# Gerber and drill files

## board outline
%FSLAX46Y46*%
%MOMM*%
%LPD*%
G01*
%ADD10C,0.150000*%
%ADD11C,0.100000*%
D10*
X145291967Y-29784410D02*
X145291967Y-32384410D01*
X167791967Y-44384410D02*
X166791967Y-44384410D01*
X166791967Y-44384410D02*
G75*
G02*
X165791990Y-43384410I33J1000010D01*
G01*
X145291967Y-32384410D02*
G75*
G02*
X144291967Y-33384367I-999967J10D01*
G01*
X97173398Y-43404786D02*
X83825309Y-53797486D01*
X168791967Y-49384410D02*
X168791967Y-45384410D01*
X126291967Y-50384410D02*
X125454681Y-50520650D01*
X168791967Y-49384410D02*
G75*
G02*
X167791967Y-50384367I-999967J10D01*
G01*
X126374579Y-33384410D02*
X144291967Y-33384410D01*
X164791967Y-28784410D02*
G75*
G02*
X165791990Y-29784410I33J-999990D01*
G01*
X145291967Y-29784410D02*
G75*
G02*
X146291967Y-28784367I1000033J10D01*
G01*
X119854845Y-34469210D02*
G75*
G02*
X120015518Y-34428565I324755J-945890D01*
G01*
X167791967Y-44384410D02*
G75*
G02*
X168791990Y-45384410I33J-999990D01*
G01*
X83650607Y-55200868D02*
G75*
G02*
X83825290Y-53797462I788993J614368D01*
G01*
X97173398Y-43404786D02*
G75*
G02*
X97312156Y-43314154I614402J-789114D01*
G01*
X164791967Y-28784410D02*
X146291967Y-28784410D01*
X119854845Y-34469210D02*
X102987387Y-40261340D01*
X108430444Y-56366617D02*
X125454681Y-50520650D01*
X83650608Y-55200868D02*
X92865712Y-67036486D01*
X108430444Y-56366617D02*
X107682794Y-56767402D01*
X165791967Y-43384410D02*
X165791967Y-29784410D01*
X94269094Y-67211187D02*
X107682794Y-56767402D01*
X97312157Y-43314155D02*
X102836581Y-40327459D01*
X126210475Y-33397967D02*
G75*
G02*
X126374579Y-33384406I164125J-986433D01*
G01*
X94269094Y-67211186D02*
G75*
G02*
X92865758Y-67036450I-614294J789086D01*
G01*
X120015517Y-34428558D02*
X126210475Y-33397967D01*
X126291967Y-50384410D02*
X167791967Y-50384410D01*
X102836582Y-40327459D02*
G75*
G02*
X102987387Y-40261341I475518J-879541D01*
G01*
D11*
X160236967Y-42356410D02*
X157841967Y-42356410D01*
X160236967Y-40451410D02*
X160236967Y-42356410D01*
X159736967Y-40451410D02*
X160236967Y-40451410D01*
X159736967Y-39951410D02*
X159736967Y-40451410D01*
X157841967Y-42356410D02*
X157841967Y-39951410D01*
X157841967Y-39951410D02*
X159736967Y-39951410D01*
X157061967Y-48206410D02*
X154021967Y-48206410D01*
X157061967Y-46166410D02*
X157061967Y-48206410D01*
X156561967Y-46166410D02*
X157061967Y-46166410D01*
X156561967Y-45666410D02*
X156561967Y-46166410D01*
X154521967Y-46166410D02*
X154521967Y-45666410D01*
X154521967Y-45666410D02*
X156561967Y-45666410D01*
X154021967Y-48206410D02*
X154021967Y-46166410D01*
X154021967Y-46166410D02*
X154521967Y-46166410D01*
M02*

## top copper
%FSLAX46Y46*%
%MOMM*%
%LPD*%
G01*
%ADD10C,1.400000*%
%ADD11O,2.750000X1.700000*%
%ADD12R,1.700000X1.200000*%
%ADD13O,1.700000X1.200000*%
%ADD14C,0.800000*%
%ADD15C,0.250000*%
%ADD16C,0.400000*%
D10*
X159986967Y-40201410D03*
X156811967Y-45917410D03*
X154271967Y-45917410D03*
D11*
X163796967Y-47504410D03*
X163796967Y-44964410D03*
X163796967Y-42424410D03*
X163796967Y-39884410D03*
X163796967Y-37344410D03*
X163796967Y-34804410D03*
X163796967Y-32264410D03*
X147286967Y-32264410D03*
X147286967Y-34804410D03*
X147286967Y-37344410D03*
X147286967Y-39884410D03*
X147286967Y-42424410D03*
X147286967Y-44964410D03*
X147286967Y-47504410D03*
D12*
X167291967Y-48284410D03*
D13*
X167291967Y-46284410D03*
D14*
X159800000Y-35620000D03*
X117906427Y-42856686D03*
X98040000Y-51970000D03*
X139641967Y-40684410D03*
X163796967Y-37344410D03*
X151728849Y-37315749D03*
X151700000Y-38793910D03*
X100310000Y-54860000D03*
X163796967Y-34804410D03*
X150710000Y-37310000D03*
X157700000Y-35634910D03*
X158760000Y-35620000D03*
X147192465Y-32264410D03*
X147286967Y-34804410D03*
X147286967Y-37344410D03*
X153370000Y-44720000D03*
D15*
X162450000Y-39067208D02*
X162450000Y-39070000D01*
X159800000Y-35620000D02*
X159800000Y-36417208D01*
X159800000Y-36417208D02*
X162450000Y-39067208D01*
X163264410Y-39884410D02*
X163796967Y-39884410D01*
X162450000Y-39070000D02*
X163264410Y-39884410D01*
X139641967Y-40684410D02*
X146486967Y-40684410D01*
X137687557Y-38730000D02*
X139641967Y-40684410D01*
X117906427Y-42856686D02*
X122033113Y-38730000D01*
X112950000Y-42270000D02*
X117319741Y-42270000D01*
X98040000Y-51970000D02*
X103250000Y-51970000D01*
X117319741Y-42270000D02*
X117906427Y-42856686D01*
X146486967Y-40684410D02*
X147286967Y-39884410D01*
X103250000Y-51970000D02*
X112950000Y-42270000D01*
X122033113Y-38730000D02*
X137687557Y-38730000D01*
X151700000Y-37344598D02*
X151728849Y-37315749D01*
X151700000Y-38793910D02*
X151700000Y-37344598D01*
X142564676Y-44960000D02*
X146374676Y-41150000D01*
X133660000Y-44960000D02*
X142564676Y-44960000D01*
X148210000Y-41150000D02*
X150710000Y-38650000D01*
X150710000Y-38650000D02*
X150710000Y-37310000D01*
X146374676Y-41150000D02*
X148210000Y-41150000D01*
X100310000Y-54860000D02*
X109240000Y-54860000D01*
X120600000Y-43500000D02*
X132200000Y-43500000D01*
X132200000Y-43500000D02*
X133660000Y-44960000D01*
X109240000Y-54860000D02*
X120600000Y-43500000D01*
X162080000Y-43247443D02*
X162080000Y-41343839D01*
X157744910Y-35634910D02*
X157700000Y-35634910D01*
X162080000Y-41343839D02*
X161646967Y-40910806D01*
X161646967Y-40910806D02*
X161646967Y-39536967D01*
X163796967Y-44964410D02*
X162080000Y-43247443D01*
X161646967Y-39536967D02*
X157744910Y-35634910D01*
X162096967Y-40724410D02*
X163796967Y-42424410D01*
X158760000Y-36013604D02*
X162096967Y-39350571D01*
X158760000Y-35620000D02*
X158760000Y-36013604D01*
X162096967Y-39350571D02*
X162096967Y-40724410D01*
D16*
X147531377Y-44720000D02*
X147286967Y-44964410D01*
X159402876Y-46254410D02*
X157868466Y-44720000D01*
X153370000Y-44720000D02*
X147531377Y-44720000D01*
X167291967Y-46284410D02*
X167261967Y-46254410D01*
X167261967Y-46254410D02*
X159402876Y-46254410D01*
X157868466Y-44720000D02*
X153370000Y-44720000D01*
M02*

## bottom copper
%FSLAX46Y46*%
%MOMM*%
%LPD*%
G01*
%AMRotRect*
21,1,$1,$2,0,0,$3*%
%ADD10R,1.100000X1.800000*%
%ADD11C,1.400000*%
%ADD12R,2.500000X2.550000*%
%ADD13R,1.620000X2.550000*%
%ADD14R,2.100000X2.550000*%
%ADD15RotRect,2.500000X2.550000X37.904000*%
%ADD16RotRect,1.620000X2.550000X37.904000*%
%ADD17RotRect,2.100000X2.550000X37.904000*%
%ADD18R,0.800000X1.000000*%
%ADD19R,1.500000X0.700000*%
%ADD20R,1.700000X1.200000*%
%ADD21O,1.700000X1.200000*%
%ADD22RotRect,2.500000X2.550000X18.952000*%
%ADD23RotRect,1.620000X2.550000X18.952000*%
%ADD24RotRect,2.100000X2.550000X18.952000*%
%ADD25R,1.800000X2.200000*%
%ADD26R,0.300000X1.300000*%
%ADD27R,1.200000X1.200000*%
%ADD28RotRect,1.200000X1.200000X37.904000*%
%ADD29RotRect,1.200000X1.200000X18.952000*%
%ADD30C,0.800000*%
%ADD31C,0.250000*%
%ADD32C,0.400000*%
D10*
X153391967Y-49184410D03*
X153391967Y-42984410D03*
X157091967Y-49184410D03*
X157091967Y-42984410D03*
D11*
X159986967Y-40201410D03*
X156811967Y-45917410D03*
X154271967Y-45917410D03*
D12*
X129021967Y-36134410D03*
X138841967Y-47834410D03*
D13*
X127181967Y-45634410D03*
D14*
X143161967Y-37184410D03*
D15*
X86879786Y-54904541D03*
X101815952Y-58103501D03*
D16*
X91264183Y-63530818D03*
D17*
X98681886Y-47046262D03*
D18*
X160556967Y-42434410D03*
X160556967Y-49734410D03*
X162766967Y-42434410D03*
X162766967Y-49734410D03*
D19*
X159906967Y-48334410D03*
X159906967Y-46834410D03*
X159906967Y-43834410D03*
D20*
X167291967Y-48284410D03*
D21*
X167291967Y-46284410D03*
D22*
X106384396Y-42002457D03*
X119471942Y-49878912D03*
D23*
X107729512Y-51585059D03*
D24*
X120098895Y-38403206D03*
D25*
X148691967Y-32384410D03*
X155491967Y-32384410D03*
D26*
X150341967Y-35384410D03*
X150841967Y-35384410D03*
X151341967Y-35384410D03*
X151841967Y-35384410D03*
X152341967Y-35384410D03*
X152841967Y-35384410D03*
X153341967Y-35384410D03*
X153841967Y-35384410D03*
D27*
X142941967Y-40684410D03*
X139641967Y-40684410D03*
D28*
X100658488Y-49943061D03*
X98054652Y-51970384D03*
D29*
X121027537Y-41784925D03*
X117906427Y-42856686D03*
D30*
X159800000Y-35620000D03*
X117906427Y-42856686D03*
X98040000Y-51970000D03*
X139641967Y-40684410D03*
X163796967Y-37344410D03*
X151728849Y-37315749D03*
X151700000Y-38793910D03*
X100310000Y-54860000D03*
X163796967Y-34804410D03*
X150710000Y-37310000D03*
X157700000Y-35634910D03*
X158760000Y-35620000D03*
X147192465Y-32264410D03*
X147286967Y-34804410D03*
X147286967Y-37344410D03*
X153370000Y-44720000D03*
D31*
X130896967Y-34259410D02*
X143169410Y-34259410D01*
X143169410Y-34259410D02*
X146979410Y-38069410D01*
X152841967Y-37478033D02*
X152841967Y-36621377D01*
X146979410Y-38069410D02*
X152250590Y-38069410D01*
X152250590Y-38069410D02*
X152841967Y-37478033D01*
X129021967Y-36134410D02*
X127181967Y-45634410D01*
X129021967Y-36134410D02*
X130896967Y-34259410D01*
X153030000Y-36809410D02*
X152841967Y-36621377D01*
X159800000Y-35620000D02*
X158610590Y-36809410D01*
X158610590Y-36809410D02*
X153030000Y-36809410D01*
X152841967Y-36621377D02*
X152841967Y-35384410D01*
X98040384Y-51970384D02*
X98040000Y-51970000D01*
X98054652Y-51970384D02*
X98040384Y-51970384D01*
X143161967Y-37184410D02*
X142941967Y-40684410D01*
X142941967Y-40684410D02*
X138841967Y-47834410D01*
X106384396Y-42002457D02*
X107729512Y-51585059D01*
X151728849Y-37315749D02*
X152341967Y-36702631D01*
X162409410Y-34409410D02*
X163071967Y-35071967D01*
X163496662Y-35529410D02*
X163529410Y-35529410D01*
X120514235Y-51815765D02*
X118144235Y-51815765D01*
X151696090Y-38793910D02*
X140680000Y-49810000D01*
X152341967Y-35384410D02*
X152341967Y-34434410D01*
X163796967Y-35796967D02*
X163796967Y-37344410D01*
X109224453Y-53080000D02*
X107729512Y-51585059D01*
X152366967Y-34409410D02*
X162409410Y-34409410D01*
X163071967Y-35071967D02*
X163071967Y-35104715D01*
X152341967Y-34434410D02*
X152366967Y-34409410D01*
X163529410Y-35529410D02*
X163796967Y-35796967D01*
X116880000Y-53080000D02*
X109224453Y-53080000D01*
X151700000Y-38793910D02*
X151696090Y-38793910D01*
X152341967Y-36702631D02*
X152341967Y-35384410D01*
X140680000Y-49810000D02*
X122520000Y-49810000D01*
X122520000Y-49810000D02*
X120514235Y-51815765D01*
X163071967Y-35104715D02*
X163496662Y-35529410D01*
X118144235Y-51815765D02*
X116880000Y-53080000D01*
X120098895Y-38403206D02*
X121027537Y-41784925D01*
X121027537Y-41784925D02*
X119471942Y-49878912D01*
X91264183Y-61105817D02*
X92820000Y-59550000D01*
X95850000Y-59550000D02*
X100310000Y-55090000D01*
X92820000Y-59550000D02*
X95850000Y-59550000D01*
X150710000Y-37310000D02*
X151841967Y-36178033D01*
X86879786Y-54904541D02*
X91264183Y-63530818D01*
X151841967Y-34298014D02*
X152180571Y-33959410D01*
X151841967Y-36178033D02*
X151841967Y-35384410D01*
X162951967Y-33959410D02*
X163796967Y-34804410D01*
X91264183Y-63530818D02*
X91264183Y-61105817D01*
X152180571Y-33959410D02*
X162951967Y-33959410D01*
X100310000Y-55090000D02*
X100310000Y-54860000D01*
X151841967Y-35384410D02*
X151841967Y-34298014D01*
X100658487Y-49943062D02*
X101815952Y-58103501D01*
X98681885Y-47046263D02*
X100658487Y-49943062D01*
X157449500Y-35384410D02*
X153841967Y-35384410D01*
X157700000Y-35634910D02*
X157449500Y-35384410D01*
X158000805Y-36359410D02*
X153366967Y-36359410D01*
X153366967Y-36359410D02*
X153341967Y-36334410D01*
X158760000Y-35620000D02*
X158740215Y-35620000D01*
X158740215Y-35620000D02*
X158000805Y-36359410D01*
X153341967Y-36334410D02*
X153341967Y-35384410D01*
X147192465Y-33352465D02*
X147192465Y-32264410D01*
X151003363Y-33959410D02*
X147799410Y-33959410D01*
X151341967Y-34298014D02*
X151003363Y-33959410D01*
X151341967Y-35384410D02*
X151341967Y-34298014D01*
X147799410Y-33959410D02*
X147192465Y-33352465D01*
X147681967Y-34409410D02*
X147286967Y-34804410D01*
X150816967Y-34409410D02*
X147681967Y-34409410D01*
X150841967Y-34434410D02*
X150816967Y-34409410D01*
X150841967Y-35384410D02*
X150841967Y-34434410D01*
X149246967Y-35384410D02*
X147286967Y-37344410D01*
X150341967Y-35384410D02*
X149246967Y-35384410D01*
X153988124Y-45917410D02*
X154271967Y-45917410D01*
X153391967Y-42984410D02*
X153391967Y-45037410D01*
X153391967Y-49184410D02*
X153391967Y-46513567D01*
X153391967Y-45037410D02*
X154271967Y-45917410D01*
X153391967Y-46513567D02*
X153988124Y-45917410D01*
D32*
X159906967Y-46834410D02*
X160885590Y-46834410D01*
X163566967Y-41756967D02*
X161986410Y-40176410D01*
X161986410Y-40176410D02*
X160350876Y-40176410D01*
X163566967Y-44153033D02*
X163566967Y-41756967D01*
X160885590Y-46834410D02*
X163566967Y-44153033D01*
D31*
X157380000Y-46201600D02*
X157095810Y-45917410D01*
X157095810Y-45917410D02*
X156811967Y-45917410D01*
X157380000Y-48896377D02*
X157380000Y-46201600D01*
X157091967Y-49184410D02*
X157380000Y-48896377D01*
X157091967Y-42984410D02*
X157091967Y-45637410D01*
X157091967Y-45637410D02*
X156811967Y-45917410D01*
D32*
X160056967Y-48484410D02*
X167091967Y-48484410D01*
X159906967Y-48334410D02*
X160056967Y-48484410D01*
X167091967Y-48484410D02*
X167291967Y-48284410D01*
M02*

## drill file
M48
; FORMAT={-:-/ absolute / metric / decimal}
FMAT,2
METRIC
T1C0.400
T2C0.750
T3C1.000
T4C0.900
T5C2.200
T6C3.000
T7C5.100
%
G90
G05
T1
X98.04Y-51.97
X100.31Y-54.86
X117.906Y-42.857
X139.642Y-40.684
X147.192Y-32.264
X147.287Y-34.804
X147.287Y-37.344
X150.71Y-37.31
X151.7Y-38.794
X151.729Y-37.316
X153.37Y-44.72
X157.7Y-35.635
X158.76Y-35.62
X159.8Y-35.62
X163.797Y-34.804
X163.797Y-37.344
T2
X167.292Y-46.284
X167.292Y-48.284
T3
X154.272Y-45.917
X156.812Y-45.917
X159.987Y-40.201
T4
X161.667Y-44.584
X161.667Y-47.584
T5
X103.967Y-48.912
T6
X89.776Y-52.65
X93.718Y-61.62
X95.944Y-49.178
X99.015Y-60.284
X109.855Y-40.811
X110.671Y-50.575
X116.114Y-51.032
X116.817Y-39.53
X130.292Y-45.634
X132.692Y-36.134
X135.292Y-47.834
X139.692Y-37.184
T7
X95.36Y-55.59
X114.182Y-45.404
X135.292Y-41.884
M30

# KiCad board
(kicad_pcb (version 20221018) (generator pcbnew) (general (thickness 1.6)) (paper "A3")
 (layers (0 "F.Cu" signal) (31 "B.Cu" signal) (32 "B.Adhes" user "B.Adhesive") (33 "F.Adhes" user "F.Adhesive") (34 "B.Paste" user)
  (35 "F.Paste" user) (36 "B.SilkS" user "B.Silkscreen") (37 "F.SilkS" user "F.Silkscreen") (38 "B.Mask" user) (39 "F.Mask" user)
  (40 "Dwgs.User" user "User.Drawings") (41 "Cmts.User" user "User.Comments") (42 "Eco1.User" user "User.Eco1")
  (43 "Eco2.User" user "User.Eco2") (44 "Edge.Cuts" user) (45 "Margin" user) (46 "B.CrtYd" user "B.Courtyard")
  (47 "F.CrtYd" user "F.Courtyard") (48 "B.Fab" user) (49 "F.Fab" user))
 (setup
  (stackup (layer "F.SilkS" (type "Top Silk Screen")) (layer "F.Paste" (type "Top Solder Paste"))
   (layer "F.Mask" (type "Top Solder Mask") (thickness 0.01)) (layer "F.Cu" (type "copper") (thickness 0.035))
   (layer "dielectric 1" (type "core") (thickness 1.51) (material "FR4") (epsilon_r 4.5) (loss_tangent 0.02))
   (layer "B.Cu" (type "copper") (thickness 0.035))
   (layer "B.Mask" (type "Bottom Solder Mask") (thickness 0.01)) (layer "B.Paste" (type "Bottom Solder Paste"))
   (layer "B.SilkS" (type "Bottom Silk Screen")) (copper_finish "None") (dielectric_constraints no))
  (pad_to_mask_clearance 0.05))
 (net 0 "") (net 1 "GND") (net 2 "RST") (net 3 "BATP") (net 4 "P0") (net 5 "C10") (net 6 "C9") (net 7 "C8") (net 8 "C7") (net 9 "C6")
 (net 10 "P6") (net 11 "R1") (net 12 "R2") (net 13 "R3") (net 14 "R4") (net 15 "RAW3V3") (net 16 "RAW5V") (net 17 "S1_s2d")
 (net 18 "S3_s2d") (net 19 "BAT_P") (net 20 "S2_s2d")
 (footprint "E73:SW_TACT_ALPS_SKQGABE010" (layer "F.Cu") (at 155.241967 46.08441 90)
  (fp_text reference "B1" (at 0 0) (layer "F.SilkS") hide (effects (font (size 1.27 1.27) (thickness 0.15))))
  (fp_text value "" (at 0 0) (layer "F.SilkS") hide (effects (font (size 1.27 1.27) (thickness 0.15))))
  (pad "1" smd rect (at -3.1 -1.85 90) (size 1.8 1.1) (layers "B.Cu" "B.Paste" "B.Mask") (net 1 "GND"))
  (pad "1" smd rect (at 3.1 -1.85 90) (size 1.8 1.1) (layers "B.Cu" "B.Paste" "B.Mask") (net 1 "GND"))
  (pad "2" smd rect (at -3.1 1.85 90) (size 1.8 1.1) (layers "B.Cu" "B.Paste" "B.Mask") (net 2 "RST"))
  (pad "2" smd rect (at 3.1 1.85 90) (size 1.8 1.1) (layers "B.Cu" "B.Paste" "B.Mask") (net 2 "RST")))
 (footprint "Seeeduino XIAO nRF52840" (layer "F.Cu") (at 155.541967 39.88441 180)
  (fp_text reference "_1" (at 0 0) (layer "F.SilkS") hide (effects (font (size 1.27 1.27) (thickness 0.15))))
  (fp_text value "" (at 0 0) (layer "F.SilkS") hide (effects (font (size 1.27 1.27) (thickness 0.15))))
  (fp_line (start -4.695 -2.472) (end -2.3 -2.472) (stroke (width 0.1) (type solid)) (layer "Edge.Cuts"))
  (fp_line (start -4.695 -0.567) (end -4.695 -2.472) (stroke (width 0.1) (type solid)) (layer "Edge.Cuts"))
  (fp_line (start -4.195 -0.567) (end -4.695 -0.567) (stroke (width 0.1) (type solid)) (layer "Edge.Cuts"))
  (fp_line (start -4.195 -0.067) (end -4.195 -0.567) (stroke (width 0.1) (type solid)) (layer "Edge.Cuts"))
  (fp_line (start -2.3 -2.472) (end -2.3 -0.067) (stroke (width 0.1) (type solid)) (layer "Edge.Cuts"))
  (fp_line (start -2.3 -0.067) (end -4.195 -0.067) (stroke (width 0.1) (type solid)) (layer "Edge.Cuts"))
  (fp_line (start -1.52 -8.322) (end 1.52 -8.322) (stroke (width 0.1) (type solid)) (layer "Edge.Cuts"))
  (fp_line (start -1.52 -6.282) (end -1.52 -8.322) (stroke (width 0.1) (type solid)) (layer "Edge.Cuts"))
  (fp_line (start -1.02 -6.282) (end -1.52 -6.282) (stroke (width 0.1) (type solid)) (layer "Edge.Cuts"))
  (fp_line (start -1.02 -5.782) (end -1.02 -6.282) (stroke (width 0.1) (type solid)) (layer "Edge.Cuts"))
  (fp_line (start 1.02 -6.282) (end 1.02 -5.782) (stroke (width 0.1) (type solid)) (layer "Edge.Cuts"))
  (fp_line (start 1.02 -5.782) (end -1.02 -5.782) (stroke (width 0.1) (type solid)) (layer "Edge.Cuts"))
  (fp_line (start 1.52 -8.322) (end 1.52 -6.282) (stroke (width 0.1) (type solid)) (layer "Edge.Cuts"))
  (fp_line (start 1.52 -6.282) (end 1.02 -6.282) (stroke (width 0.1) (type solid)) (layer "Edge.Cuts"))
  (pad "" thru_hole circle (at -4.445 -0.317) (size 1.4 1.4) (drill 1) (layers "*.Cu" "*.Mask") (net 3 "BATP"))
  (pad "" thru_hole circle (at -1.27 -6.033) (size 1.4 1.4) (drill 1) (layers "*.Cu" "*.Mask") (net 2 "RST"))
  (pad "" thru_hole circle (at 1.27 -6.033) (size 1.4 1.4) (drill 1) (layers "*.Cu" "*.Mask") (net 1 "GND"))
  (pad "1" smd oval (at -8.255 -7.62 180) (size 2.75 1.7) (layers "F.Cu" "F.Paste" "F.Mask") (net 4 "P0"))
  (pad "2" smd oval (at -8.255 -5.08 180) (size 2.75 1.7) (layers "F.Cu" "F.Paste" "F.Mask") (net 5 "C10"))
  (pad "3" smd oval (at -8.255 -2.54 180) (size 2.75 1.7) (layers "F.Cu" "F.Paste" "F.Mask") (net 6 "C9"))
  (pad "4" smd oval (at -8.255 0 180) (size 2.75 1.7) (layers "F.Cu" "F.Paste" "F.Mask") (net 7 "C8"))
  (pad "5" smd oval (at -8.255 2.54 180) (size 2.75 1.7) (layers "F.Cu" "F.Paste" "F.Mask") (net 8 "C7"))
  (pad "6" smd oval (at -8.255 5.08 180) (size 2.75 1.7) (layers "F.Cu" "F.Paste" "F.Mask") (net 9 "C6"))
  (pad "7" smd oval (at -8.255 7.62 180) (size 2.75 1.7) (layers "F.Cu" "F.Paste" "F.Mask") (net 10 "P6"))
  (pad "8" smd oval (at 8.255 7.62 180) (size 2.75 1.7) (layers "F.Cu" "F.Paste" "F.Mask") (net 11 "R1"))
  (pad "9" smd oval (at 8.255 5.08 180) (size 2.75 1.7) (layers "F.Cu" "F.Paste" "F.Mask") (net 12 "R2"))
  (pad "10" smd oval (at 8.255 2.54 180) (size 2.75 1.7) (layers "F.Cu" "F.Paste" "F.Mask") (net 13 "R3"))
  (pad "11" smd oval (at 8.255 0 180) (size 2.75 1.7) (layers "F.Cu" "F.Paste" "F.Mask") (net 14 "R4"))
  (pad "12" smd oval (at 8.255 -2.54 180) (size 2.75 1.7) (layers "F.Cu" "F.Paste" "F.Mask") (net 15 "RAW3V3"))
  (pad "13" smd oval (at 8.255 -5.08 180) (size 2.75 1.7) (layers "F.Cu" "F.Paste" "F.Mask") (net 1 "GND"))
  (pad "14" smd oval (at 8.255 -7.62 180) (size 2.75 1.7) (layers "F.Cu" "F.Paste" "F.Mask") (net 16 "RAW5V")))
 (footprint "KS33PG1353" (layer "F.Cu") (at 135.291967 41.88441)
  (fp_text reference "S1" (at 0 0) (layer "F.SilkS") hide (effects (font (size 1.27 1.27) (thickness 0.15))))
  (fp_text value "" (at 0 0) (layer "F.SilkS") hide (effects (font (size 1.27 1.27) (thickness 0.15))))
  (pad "" np_thru_hole circle (at -5 3.75) (size 3 3) (drill 3) (layers "*.Cu" "*.Mask"))
  (pad "" np_thru_hole circle (at -2.6 -5.75) (size 3 3) (drill 3) (layers "*.Cu" "*.Mask"))
  (pad "" np_thru_hole circle (at 0 0) (size 5.1 5.1) (drill 5.1) (layers "*.Cu" "*.Mask"))
  (pad "" np_thru_hole circle (at 0 5.95) (size 3 3) (drill 3) (layers "*.Cu" "*.Mask"))
  (pad "" np_thru_hole circle (at 4.4 -4.7) (size 3 3) (drill 3) (layers "*.Cu" "*.Mask"))
  (pad "1" smd rect (at -6.27 -5.75) (size 2.5 2.55) (layers "B.Cu" "B.Paste" "B.Mask") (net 7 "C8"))
  (pad "1" smd rect (at 3.55 5.95) (size 2.5 2.55) (layers "B.Cu" "B.Paste" "B.Mask") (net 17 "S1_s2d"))
  (pad "2" smd rect (at -8.11 3.75) (size 1.62 2.55) (layers "B.Cu" "B.Paste" "B.Mask") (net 7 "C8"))
  (pad "2" smd rect (at 7.87 -4.7) (size 2.1 2.55) (layers "B.Cu" "B.Paste" "B.Mask") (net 17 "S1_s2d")))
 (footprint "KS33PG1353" (layer "F.Cu") (at 95.359531 55.589614 37.904)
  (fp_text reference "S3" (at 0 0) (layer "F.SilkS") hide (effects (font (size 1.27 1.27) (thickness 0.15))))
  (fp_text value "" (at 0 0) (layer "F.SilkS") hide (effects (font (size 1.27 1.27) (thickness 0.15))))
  (pad "" np_thru_hole circle (at -5 3.75) (size 3 3) (drill 3) (layers "*.Cu" "*.Mask"))
  (pad "" np_thru_hole circle (at -2.6 -5.75) (size 3 3) (drill 3) (layers "*.Cu" "*.Mask"))
  (pad "" np_thru_hole circle (at 0 0) (size 5.1 5.1) (drill 5.1) (layers "*.Cu" "*.Mask"))
  (pad "" np_thru_hole circle (at 0 5.95) (size 3 3) (drill 3) (layers "*.Cu" "*.Mask"))
  (pad "" np_thru_hole circle (at 4.4 -4.7) (size 3 3) (drill 3) (layers "*.Cu" "*.Mask"))
  (pad "1" smd rect (at -6.27 -5.75 37.904) (size 2.5 2.55) (layers "B.Cu" "B.Paste" "B.Mask") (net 9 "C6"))
  (pad "1" smd rect (at 3.55 5.95 37.904) (size 2.5 2.55) (layers "B.Cu" "B.Paste" "B.Mask") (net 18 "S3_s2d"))
  (pad "2" smd rect (at -8.11 3.75 37.904) (size 1.62 2.55) (layers "B.Cu" "B.Paste" "B.Mask") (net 9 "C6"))
  (pad "2" smd rect (at 7.87 -4.7 37.904) (size 2.1 2.55) (layers "B.Cu" "B.Paste" "B.Mask") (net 18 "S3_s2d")))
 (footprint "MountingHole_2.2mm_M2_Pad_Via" (layer "F.Cu") (at 103.967424 48.91199 18.952)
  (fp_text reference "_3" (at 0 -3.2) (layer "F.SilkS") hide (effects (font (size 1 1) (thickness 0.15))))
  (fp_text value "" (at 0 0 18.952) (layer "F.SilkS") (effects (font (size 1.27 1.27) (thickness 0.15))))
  (pad "" np_thru_hole circle (at 0 0) (size 2.2 2.2) (drill 2.2) (layers "*.Cu" "*.Mask")))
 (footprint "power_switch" (layer "F.Cu") (at 161.641967 46.08441)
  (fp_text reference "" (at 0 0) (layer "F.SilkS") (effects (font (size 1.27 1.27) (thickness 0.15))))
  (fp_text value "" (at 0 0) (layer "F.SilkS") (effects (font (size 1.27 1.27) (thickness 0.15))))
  (pad "" smd rect (at -1.085 -3.65 270) (size 1 0.8) (layers "B.Cu" "B.Paste" "B.Mask"))
  (pad "" smd rect (at -1.085 3.65 270) (size 1 0.8) (layers "B.Cu" "B.Paste" "B.Mask"))
  (pad "" np_thru_hole circle (at 0.025 -1.5 90) (size 0.9 0.9) (drill 0.9) (layers "*.Cu" "*.Mask"))
  (pad "" np_thru_hole circle (at 0.025 1.5 90) (size 0.9 0.9) (drill 0.9) (layers "*.Cu" "*.Mask"))
  (pad "" smd rect (at 1.125 -3.65 270) (size 1 0.8) (layers "B.Cu" "B.Paste" "B.Mask"))
  (pad "" smd rect (at 1.125 3.65 270) (size 1 0.8) (layers "B.Cu" "B.Paste" "B.Mask"))
  (pad "4" smd rect (at -1.735 2.25 270) (size 0.7 1.5) (layers "B.Cu" "B.Paste" "B.Mask") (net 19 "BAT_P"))
  (pad "5" smd rect (at -1.735 0.75 270) (size 0.7 1.5) (layers "B.Cu" "B.Paste" "B.Mask") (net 3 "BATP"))
  (pad "6" smd rect (at -1.735 -2.25 270) (size 0.7 1.5) (layers "B.Cu" "B.Paste" "B.Mask")))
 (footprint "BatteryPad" (layer "F.Cu") (at 167.291967 47.28441 90)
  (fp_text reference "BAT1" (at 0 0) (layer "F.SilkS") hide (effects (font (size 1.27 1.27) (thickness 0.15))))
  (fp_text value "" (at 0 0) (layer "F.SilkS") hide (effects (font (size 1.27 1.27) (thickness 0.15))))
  (pad "1" thru_hole rect (at -1 0 90) (size 1.2 1.7) (drill 0.75) (layers "*.Cu" "*.Mask") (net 19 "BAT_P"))
  (pad "2" thru_hole oval (at 1 0 90) (size 1.2 1.7) (drill 0.75) (layers "*.Cu" "*.Mask") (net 1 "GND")))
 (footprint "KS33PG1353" (layer "F.Cu") (at 114.181967 45.40441 18.952)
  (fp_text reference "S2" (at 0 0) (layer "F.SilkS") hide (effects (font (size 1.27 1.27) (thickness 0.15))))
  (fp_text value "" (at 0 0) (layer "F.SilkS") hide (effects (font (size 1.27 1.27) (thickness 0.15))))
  (pad "" np_thru_hole circle (at -5 3.75) (size 3 3) (drill 3) (layers "*.Cu" "*.Mask"))
  (pad "" np_thru_hole circle (at -2.6 -5.75) (size 3 3) (drill 3) (layers "*.Cu" "*.Mask"))
  (pad "" np_thru_hole circle (at 0 0) (size 5.1 5.1) (drill 5.1) (layers "*.Cu" "*.Mask"))
  (pad "" np_thru_hole circle (at 0 5.95) (size 3 3) (drill 3) (layers "*.Cu" "*.Mask"))
  (pad "" np_thru_hole circle (at 4.4 -4.7) (size 3 3) (drill 3) (layers "*.Cu" "*.Mask"))
  (pad "1" smd rect (at -6.27 -5.75 18.952) (size 2.5 2.55) (layers "B.Cu" "B.Paste" "B.Mask") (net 8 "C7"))
  (pad "1" smd rect (at 3.55 5.95 18.952) (size 2.5 2.55) (layers "B.Cu" "B.Paste" "B.Mask") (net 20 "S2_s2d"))
  (pad "2" smd rect (at -8.11 3.75 18.952) (size 1.62 2.55) (layers "B.Cu" "B.Paste" "B.Mask") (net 8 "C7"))
  (pad "2" smd rect (at 7.87 -4.7 18.952) (size 2.1 2.55) (layers "B.Cu" "B.Paste" "B.Mask") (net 20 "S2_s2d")))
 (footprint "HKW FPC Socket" (layer "B.Cu") (at 152.091967 32.38441)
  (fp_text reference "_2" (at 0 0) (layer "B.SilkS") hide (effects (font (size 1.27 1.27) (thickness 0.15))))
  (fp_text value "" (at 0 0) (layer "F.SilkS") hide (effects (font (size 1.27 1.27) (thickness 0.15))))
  (pad "" smd rect (at -3.4 0) (size 1.8 2.2) (layers "B.Cu" "B.Paste" "B.Mask"))
  (pad "" smd rect (at 3.4 0) (size 1.8 2.2) (layers "B.Cu" "B.Paste" "B.Mask"))
  (pad "1" smd rect (at -1.75 3) (size 0.3 1.3) (layers "B.Cu" "B.Paste" "B.Mask") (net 13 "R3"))
  (pad "2" smd rect (at -1.25 3) (size 0.3 1.3) (layers "B.Cu" "B.Paste" "B.Mask") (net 12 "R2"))
  (pad "3" smd rect (at -0.75 3) (size 0.3 1.3) (layers "B.Cu" "B.Paste" "B.Mask") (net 11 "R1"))
  (pad "4" smd rect (at -0.25 3) (size 0.3 1.3) (layers "B.Cu" "B.Paste" "B.Mask") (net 9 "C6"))
  (pad "5" smd rect (at 0.25 3) (size 0.3 1.3) (layers "B.Cu" "B.Paste" "B.Mask") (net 8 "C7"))
  (pad "6" smd rect (at 0.75 3) (size 0.3 1.3) (layers "B.Cu" "B.Paste" "B.Mask") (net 7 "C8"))
  (pad "7" smd rect (at 1.25 3) (size 0.3 1.3) (layers "B.Cu" "B.Paste" "B.Mask") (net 6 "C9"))
  (pad "8" smd rect (at 1.75 3) (size 0.3 1.3) (layers "B.Cu" "B.Paste" "B.Mask") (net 5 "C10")))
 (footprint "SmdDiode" (layer "B.Cu") (at 135.291967 41.88441)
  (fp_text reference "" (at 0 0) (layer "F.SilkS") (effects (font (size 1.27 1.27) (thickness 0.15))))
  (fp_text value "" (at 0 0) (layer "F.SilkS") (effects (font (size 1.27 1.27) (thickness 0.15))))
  (pad "1" smd rect (at 7.65 -1.2) (size 1.2 1.2) (layers "B.Cu" "B.Paste" "B.Mask") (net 17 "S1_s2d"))
  (pad "2" smd rect (at 4.35 -1.2) (size 1.2 1.2) (layers "B.Cu" "B.Paste" "B.Mask") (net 14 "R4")))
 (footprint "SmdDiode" (layer "B.Cu") (at 95.359531 55.589614 37.904)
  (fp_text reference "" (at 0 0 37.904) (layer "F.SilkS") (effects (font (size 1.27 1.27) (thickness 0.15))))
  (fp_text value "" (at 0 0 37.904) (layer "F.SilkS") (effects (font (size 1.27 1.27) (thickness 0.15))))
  (pad "1" smd rect (at 7.65 -1.2 37.904) (size 1.2 1.2) (layers "B.Cu" "B.Paste" "B.Mask") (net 18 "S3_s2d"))
  (pad "2" smd rect (at 4.35 -1.2 37.904) (size 1.2 1.2) (layers "B.Cu" "B.Paste" "B.Mask") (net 14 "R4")))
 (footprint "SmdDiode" (layer "B.Cu") (at 114.181967 45.40441 18.952)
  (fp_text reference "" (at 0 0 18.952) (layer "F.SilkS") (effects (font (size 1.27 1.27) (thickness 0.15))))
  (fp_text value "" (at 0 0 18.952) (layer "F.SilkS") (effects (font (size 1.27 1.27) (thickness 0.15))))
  (pad "1" smd rect (at 7.65 -1.2 18.952) (size 1.2 1.2) (layers "B.Cu" "B.Paste" "B.Mask") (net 20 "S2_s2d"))
  (pad "2" smd rect (at 4.35 -1.2 18.952) (size 1.2 1.2) (layers "B.Cu" "B.Paste" "B.Mask") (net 14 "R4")))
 (gr_line (start 145.291967 29.78441) (end 145.291967 32.38441) (stroke (width 0.15) (type solid)) (layer "Edge.Cuts"))
 (gr_line (start 167.791967 44.38441) (end 166.791967 44.38441) (stroke (width 0.15) (type solid)) (layer "Edge.Cuts"))
 (gr_arc (start 166.791967 44.38441) (mid 166.08486 44.091517) (end 165.791967 43.38441) (stroke (width 0.15) (type solid))
  (layer "Edge.Cuts"))
 (gr_arc (start 145.291967 32.38441) (mid 144.999074 33.091517) (end 144.291967 33.38441) (stroke (width 0.15) (type solid))
  (layer "Edge.Cuts"))
 (gr_line (start 97.173398 43.404786) (end 83.825309 53.797486) (stroke (width 0.15) (type solid)) (layer "Edge.Cuts"))
 (gr_line (start 168.791967 49.38441) (end 168.791967 45.38441) (stroke (width 0.15) (type solid)) (layer "Edge.Cuts"))
 (gr_line (start 126.291967 50.38441) (end 125.454681 50.52065) (stroke (width 0.15) (type solid)) (layer "Edge.Cuts"))
 (gr_arc (start 168.791967 49.38441) (mid 168.499074 50.091517) (end 167.791967 50.38441) (stroke (width 0.15) (type solid))
  (layer "Edge.Cuts"))
 (gr_line (start 126.374579 33.38441) (end 144.291967 33.38441) (stroke (width 0.15) (type solid)) (layer "Edge.Cuts"))
 (gr_arc (start 164.791967 28.78441) (mid 165.499074 29.077303) (end 165.791967 29.78441) (stroke (width 0.15) (type solid))
  (layer "Edge.Cuts"))
 (gr_arc (start 145.291967 29.78441) (mid 145.58486 29.077303) (end 146.291967 28.78441) (stroke (width 0.15) (type solid))
  (layer "Edge.Cuts"))
 (gr_arc (start 119.854845 34.46921) (mid 119.934337 34.44555) (end 120.015517 34.428558) (stroke (width 0.15) (type solid))
  (layer "Edge.Cuts"))
 (gr_arc (start 167.791967 44.38441) (mid 168.499074 44.677303) (end 168.791967 45.38441) (stroke (width 0.15) (type solid))
  (layer "Edge.Cuts"))
 (gr_arc (start 83.650607 55.200868) (mid 83.447308 54.462995) (end 83.825309 53.797486) (stroke (width 0.15) (type solid))
  (layer "Edge.Cuts"))
 (gr_arc (start 97.173398 43.404786) (mid 97.240897 43.356591) (end 97.312157 43.314155) (stroke (width 0.15) (type solid))
  (layer "Edge.Cuts"))
 (gr_line (start 164.791967 28.78441) (end 146.291967 28.78441) (stroke (width 0.15) (type solid)) (layer "Edge.Cuts"))
 (gr_line (start 119.854845 34.46921) (end 102.987387 40.26134) (stroke (width 0.15) (type solid)) (layer "Edge.Cuts"))
 (gr_line (start 108.430444 56.366617) (end 125.454681 50.52065) (stroke (width 0.15) (type solid)) (layer "Edge.Cuts"))
 (gr_line (start 83.650608 55.200868) (end 92.865712 67.036486) (stroke (width 0.15) (type solid)) (layer "Edge.Cuts"))
 (gr_line (start 108.430444 56.366617) (end 107.682794 56.767402) (stroke (width 0.15) (type solid)) (layer "Edge.Cuts"))
 (gr_line (start 165.791967 43.38441) (end 165.791967 29.78441) (stroke (width 0.15) (type solid)) (layer "Edge.Cuts"))
 (gr_line (start 94.269094 67.211187) (end 107.682794 56.767402) (stroke (width 0.15) (type solid)) (layer "Edge.Cuts"))
 (gr_line (start 97.312157 43.314155) (end 102.836581 40.327459) (stroke (width 0.15) (type solid)) (layer "Edge.Cuts"))
 (gr_arc (start 126.210475 33.397967) (mid 126.292247 33.387805) (end 126.374579 33.38441) (stroke (width 0.15) (type solid))
  (layer "Edge.Cuts"))
 (gr_arc (start 94.269094 67.211186) (mid 93.531221 67.414486) (end 92.865712 67.036486) (stroke (width 0.15) (type solid))
  (layer "Edge.Cuts"))
 (gr_line (start 120.015517 34.428558) (end 126.210475 33.397967) (stroke (width 0.15) (type solid)) (layer "Edge.Cuts"))
 (gr_line (start 126.291967 50.38441) (end 167.791967 50.38441) (stroke (width 0.15) (type solid)) (layer "Edge.Cuts"))
 (gr_arc (start 102.836582 40.327459) (mid 102.910621 40.29129) (end 102.987387 40.26134) (stroke (width 0.15) (type solid))
  (layer "Edge.Cuts"))
 (segment (start 162.45 39.067208) (end 162.45 39.07) (width 0.25) (layer "F.Cu") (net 7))
 (segment (start 159.8 35.62) (end 159.8 36.417208) (width 0.25) (layer "F.Cu") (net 7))
 (segment (start 159.8 36.417208) (end 162.45 39.067208) (width 0.25) (layer "F.Cu") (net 7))
 (segment (start 163.26441 39.88441) (end 163.796967 39.88441) (width 0.25) (layer "F.Cu") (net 7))
 (segment (start 162.45 39.07) (end 163.26441 39.88441) (width 0.25) (layer "F.Cu") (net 7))
 (via (at 159.8 35.62) (size 0.8) (drill 0.4) (layers "F.Cu" "B.Cu") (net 7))
 (segment (start 130.896967 34.25941) (end 143.16941 34.25941) (width 0.25) (layer "B.Cu") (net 7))
 (segment (start 143.16941 34.25941) (end 146.97941 38.06941) (width 0.25) (layer "B.Cu") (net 7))
 (segment (start 152.841967 37.478033) (end 152.841967 36.621377) (width 0.25) (layer "B.Cu") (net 7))
 (segment (start 146.97941 38.06941) (end 152.25059 38.06941) (width 0.25) (layer "B.Cu") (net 7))
 (segment (start 152.25059 38.06941) (end 152.841967 37.478033) (width 0.25) (layer "B.Cu") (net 7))
 (segment (start 129.021967 36.13441) (end 127.181967 45.63441) (width 0.25) (layer "B.Cu") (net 7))
 (segment (start 129.021967 36.13441) (end 130.896967 34.25941) (width 0.25) (layer "B.Cu") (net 7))
 (segment (start 153.03 36.80941) (end 152.841967 36.621377) (width 0.25) (layer "B.Cu") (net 7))
 (segment (start 159.8 35.62) (end 158.61059 36.80941) (width 0.25) (layer "B.Cu") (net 7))
 (segment (start 158.61059 36.80941) (end 153.03 36.80941) (width 0.25) (layer "B.Cu") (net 7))
 (segment (start 152.841967 36.621377) (end 152.841967 35.38441) (width 0.25) (layer "B.Cu") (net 7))
 (segment (start 139.641967 40.68441) (end 146.486967 40.68441) (width 0.25) (layer "F.Cu") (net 14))
 (segment (start 137.687557 38.73) (end 139.641967 40.68441) (width 0.25) (layer "F.Cu") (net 14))
 (segment (start 117.906427 42.856686) (end 122.033113 38.73) (width 0.25) (layer "F.Cu") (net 14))
 (segment (start 112.95 42.27) (end 117.319741 42.27) (width 0.25) (layer "F.Cu") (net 14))
 (segment (start 98.04 51.97) (end 103.25 51.97) (width 0.25) (layer "F.Cu") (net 14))
 (segment (start 117.319741 42.27) (end 117.906427 42.856686) (width 0.25) (layer "F.Cu") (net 14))
 (segment (start 146.486967 40.68441) (end 147.286967 39.88441) (width 0.25) (layer "F.Cu") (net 14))
 (segment (start 103.25 51.97) (end 112.95 42.27) (width 0.25) (layer "F.Cu") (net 14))
 (segment (start 122.033113 38.73) (end 137.687557 38.73) (width 0.25) (layer "F.Cu") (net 14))
 (via (at 117.906427 42.856686) (size 0.8) (drill 0.4) (layers "F.Cu" "B.Cu") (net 14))
 (via (at 98.04 51.97) (size 0.8) (drill 0.4) (layers "F.Cu" "B.Cu") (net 14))
 (via (at 139.641967 40.68441) (size 0.8) (drill 0.4) (layers "F.Cu" "B.Cu") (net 14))
 (segment (start 98.040384 51.970384) (end 98.04 51.97) (width 0.25) (layer "B.Cu") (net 14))
 (segment (start 98.054652 51.970384) (end 98.040384 51.970384) (width 0.25) (layer "B.Cu") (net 14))
 (segment (start 143.161967 37.18441) (end 142.941967 40.68441) (width 0.25) (layer "B.Cu") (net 17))
 (segment (start 142.941967 40.68441) (end 138.841967 47.83441) (width 0.25) (layer "B.Cu") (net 17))
 (segment (start 151.7 37.344598) (end 151.728849 37.315749) (width 0.25) (layer "F.Cu") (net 8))
 (segment (start 151.7 38.79391) (end 151.7 37.344598) (width 0.25) (layer "F.Cu") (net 8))
 (via (at 163.796967 37.34441) (size 0.8) (drill 0.4) (layers "F.Cu" "B.Cu") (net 8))
 (via (at 151.728849 37.315749) (size 0.8) (drill 0.4) (layers "F.Cu" "B.Cu") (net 8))
 (via (at 151.7 38.79391) (size 0.8) (drill 0.4) (layers "F.Cu" "B.Cu") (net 8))
 (segment (start 106.384396 42.002457) (end 107.729512 51.585059) (width 0.25) (layer "B.Cu") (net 8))
 (segment (start 151.728849 37.315749) (end 152.341967 36.702631) (width 0.25) (layer "B.Cu") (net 8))
 (segment (start 162.40941 34.40941) (end 163.071967 35.071967) (width 0.25) (layer "B.Cu") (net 8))
 (segment (start 163.496662 35.52941) (end 163.52941 35.52941) (width 0.25) (layer "B.Cu") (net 8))
 (segment (start 120.514235 51.815765) (end 118.144235 51.815765) (width 0.25) (layer "B.Cu") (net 8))
 (segment (start 151.69609 38.79391) (end 140.68 49.81) (width 0.25) (layer "B.Cu") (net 8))
 (segment (start 152.341967 35.38441) (end 152.341967 34.43441) (width 0.25) (layer "B.Cu") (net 8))
 (segment (start 163.796967 35.796967) (end 163.796967 37.34441) (width 0.25) (layer "B.Cu") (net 8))
 (segment (start 109.224453 53.08) (end 107.729512 51.585059) (width 0.25) (layer "B.Cu") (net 8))
 (segment (start 152.366967 34.40941) (end 162.40941 34.40941) (width 0.25) (layer "B.Cu") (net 8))
 (segment (start 163.071967 35.071967) (end 163.071967 35.104715) (width 0.25) (layer "B.Cu") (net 8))
 (segment (start 152.341967 34.43441) (end 152.366967 34.40941) (width 0.25) (layer "B.Cu") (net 8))
 (segment (start 163.52941 35.52941) (end 163.796967 35.796967) (width 0.25) (layer "B.Cu") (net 8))
 (segment (start 116.88 53.08) (end 109.224453 53.08) (width 0.25) (layer "B.Cu") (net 8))
 (segment (start 151.7 38.79391) (end 151.69609 38.79391) (width 0.25) (layer "B.Cu") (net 8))
 (segment (start 152.341967 36.702631) (end 152.341967 35.38441) (width 0.25) (layer "B.Cu") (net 8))
 (segment (start 140.68 49.81) (end 122.52 49.81) (width 0.25) (layer "B.Cu") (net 8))
 (segment (start 122.52 49.81) (end 120.514235 51.815765) (width 0.25) (layer "B.Cu") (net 8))
 (segment (start 163.071967 35.104715) (end 163.496662 35.52941) (width 0.25) (layer "B.Cu") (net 8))
 (segment (start 118.144235 51.815765) (end 116.88 53.08) (width 0.25) (layer "B.Cu") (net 8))
 (segment (start 120.098895 38.403206) (end 121.027537 41.784925) (width 0.25) (layer "B.Cu") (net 20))
 (segment (start 121.027537 41.784925) (end 119.471942 49.878912) (width 0.25) (layer "B.Cu") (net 20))
 (segment (start 142.564676 44.96) (end 146.374676 41.15) (width 0.25) (layer "F.Cu") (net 9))
 (segment (start 133.66 44.96) (end 142.564676 44.96) (width 0.25) (layer "F.Cu") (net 9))
 (segment (start 148.21 41.15) (end 150.71 38.65) (width 0.25) (layer "F.Cu") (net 9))
 (segment (start 150.71 38.65) (end 150.71 37.31) (width 0.25) (layer "F.Cu") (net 9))
 (segment (start 146.374676 41.15) (end 148.21 41.15) (width 0.25) (layer "F.Cu") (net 9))
 (segment (start 100.31 54.86) (end 109.24 54.86) (width 0.25) (layer "F.Cu") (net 9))
 (segment (start 120.6 43.5) (end 132.2 43.5) (width 0.25) (layer "F.Cu") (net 9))
 (segment (start 132.2 43.5) (end 133.66 44.96) (width 0.25) (layer "F.Cu") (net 9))
 (segment (start 109.24 54.86) (end 120.6 43.5) (width 0.25) (layer "F.Cu") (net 9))
 (via (at 100.31 54.86) (size 0.8) (drill 0.4) (layers "F.Cu" "B.Cu") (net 9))
 (via (at 163.796967 34.80441) (size 0.8) (drill 0.4) (layers "F.Cu" "B.Cu") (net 9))
 (via (at 150.71 37.31) (size 0.8) (drill 0.4) (layers "F.Cu" "B.Cu") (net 9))
 (segment (start 91.264183 61.105817) (end 92.82 59.55) (width 0.25) (layer "B.Cu") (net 9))
 (segment (start 95.85 59.55) (end 100.31 55.09) (width 0.25) (layer "B.Cu") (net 9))
 (segment (start 92.82 59.55) (end 95.85 59.55) (width 0.25) (layer "B.Cu") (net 9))
 (segment (start 150.71 37.31) (end 151.841967 36.178033) (width 0.25) (layer "B.Cu") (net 9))
 (segment (start 86.879786 54.904541) (end 91.264183 63.530818) (width 0.25) (layer "B.Cu") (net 9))
 (segment (start 151.841967 34.298014) (end 152.180571 33.95941) (width 0.25) (layer "B.Cu") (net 9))
 (segment (start 151.841967 36.178033) (end 151.841967 35.38441) (width 0.25) (layer "B.Cu") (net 9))
 (segment (start 162.951967 33.95941) (end 163.796967 34.80441) (width 0.25) (layer "B.Cu") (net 9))
 (segment (start 91.264183 63.530818) (end 91.264183 61.105817) (width 0.25) (layer "B.Cu") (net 9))
 (segment (start 152.180571 33.95941) (end 162.951967 33.95941) (width 0.25) (layer "B.Cu") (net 9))
 (segment (start 100.31 55.09) (end 100.31 54.86) (width 0.25) (layer "B.Cu") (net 9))
 (segment (start 151.841967 35.38441) (end 151.841967 34.298014) (width 0.25) (layer "B.Cu") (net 9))
 (segment (start 100.658487 49.943062) (end 101.815952 58.103501) (width 0.25) (layer "B.Cu") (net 18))
 (segment (start 98.681885 47.046263) (end 100.658487 49.943062) (width 0.25) (layer "B.Cu") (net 18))
 (segment (start 162.08 43.247443) (end 162.08 41.343839) (width 0.25) (layer "F.Cu") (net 5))
 (segment (start 157.74491 35.63491) (end 157.7 35.63491) (width 0.25) (layer "F.Cu") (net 5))
 (segment (start 162.08 41.343839) (end 161.646967 40.910806) (width 0.25) (layer "F.Cu") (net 5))
 (segment (start 161.646967 40.910806) (end 161.646967 39.536967) (width 0.25) (layer "F.Cu") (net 5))
 (segment (start 163.796967 44.96441) (end 162.08 43.247443) (width 0.25) (layer "F.Cu") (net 5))
 (segment (start 161.646967 39.536967) (end 157.74491 35.63491) (width 0.25) (layer "F.Cu") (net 5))
 (via (at 157.7 35.63491) (size 0.8) (drill 0.4) (layers "F.Cu" "B.Cu") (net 5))
 (segment (start 157.4495 35.38441) (end 153.841967 35.38441) (width 0.25) (layer "B.Cu") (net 5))
 (segment (start 157.7 35.63491) (end 157.4495 35.38441) (width 0.25) (layer "B.Cu") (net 5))
 (segment (start 162.096967 40.72441) (end 163.796967 42.42441) (width 0.25) (layer "F.Cu") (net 6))
 (segment (start 158.76 36.013604) (end 162.096967 39.350571) (width 0.25) (layer "F.Cu") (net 6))
 (segment (start 158.76 35.62) (end 158.76 36.013604) (width 0.25) (layer "F.Cu") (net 6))
 (segment (start 162.096967 39.350571) (end 162.096967 40.72441) (width 0.25) (layer "F.Cu") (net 6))
 (via (at 158.76 35.62) (size 0.8) (drill 0.4) (layers "F.Cu" "B.Cu") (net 6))
 (segment (start 158.000805 36.35941) (end 153.366967 36.35941) (width 0.25) (layer "B.Cu") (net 6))
 (segment (start 153.366967 36.35941) (end 153.341967 36.33441) (width 0.25) (layer "B.Cu") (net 6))
 (segment (start 158.76 35.62) (end 158.740215 35.62) (width 0.25) (layer "B.Cu") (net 6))
 (segment (start 158.740215 35.62) (end 158.000805 36.35941) (width 0.25) (layer "B.Cu") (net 6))
 (segment (start 153.341967 36.33441) (end 153.341967 35.38441) (width 0.25) (layer "B.Cu") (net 6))
 (via (at 147.192465 32.26441) (size 0.8) (drill 0.4) (layers "F.Cu" "B.Cu") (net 11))
 (segment (start 147.192465 33.352465) (end 147.192465 32.26441) (width 0.25) (layer "B.Cu") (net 11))
 (segment (start 151.003363 33.95941) (end 147.79941 33.95941) (width 0.25) (layer "B.Cu") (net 11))
 (segment (start 151.341967 34.298014) (end 151.003363 33.95941) (width 0.25) (layer "B.Cu") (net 11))
 (segment (start 151.341967 35.38441) (end 151.341967 34.298014) (width 0.25) (layer "B.Cu") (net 11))
 (segment (start 147.79941 33.95941) (end 147.192465 33.352465) (width 0.25) (layer "B.Cu") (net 11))
 (via (at 147.286967 34.80441) (size 0.8) (drill 0.4) (layers "F.Cu" "B.Cu") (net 12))
 (segment (start 147.681967 34.40941) (end 147.286967 34.80441) (width 0.25) (layer "B.Cu") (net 12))
 (segment (start 150.816967 34.40941) (end 147.681967 34.40941) (width 0.25) (layer "B.Cu") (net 12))
 (segment (start 150.841967 34.43441) (end 150.816967 34.40941) (width 0.25) (layer "B.Cu") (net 12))
 (segment (start 150.841967 35.38441) (end 150.841967 34.43441) (width 0.25) (layer "B.Cu") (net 12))
 (via (at 147.286967 37.34441) (size 0.8) (drill 0.4) (layers "F.Cu" "B.Cu") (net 13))
 (segment (start 149.246967 35.38441) (end 147.286967 37.34441) (width 0.25) (layer "B.Cu") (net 13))
 (segment (start 150.341967 35.38441) (end 149.246967 35.38441) (width 0.25) (layer "B.Cu") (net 13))
 (segment (start 147.531377 44.72) (end 147.286967 44.96441) (width 0.4) (layer "F.Cu") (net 1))
 (segment (start 159.402876 46.25441) (end 157.868466 44.72) (width 0.4) (layer "F.Cu") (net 1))
 (segment (start 153.37 44.72) (end 147.531377 44.72) (width 0.4) (layer "F.Cu") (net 1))
 (segment (start 167.291967 46.28441) (end 167.261967 46.25441) (width 0.4) (layer "F.Cu") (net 1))
 (segment (start 167.261967 46.25441) (end 159.402876 46.25441) (width 0.4) (layer "F.Cu") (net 1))
 (segment (start 157.868466 44.72) (end 153.37 44.72) (width 0.4) (layer "F.Cu") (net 1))
 (via (at 153.37 44.72) (size 0.8) (drill 0.4) (layers "F.Cu" "B.Cu") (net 1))
 (segment (start 153.988124 45.91741) (end 154.271967 45.91741) (width 0.25) (layer "B.Cu") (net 1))
 (segment (start 153.391967 42.98441) (end 153.391967 45.03741) (width 0.25) (layer "B.Cu") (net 1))
 (segment (start 153.391967 49.18441) (end 153.391967 46.513567) (width 0.25) (layer "B.Cu") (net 1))
 (segment (start 153.391967 45.03741) (end 154.271967 45.91741) (width 0.25) (layer "B.Cu") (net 1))
 (segment (start 153.391967 46.513567) (end 153.988124 45.91741) (width 0.25) (layer "B.Cu") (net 1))
 (segment (start 159.906967 46.83441) (end 160.88559 46.83441) (width 0.4) (layer "B.Cu") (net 3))
 (segment (start 163.566967 41.756967) (end 161.98641 40.17641) (width 0.4) (layer "B.Cu") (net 3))
 (segment (start 161.98641 40.17641) (end 160.350876 40.17641) (width 0.4) (layer "B.Cu") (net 3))
 (segment (start 163.566967 44.153033) (end 163.566967 41.756967) (width 0.4) (layer "B.Cu") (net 3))
 (segment (start 160.88559 46.83441) (end 163.566967 44.153033) (width 0.4) (layer "B.Cu") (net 3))
 (segment (start 157.38 46.2016) (end 157.09581 45.91741) (width 0.25) (layer "B.Cu") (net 2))
 (segment (start 157.09581 45.91741) (end 156.811967 45.91741) (width 0.25) (layer "B.Cu") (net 2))
 (segment (start 157.38 48.896377) (end 157.38 46.2016) (width 0.25) (layer "B.Cu") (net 2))
 (segment (start 157.091967 49.18441) (end 157.38 48.896377) (width 0.25) (layer "B.Cu") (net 2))
 (segment (start 157.091967 42.98441) (end 157.091967 45.63741) (width 0.25) (layer "B.Cu") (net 2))
 (segment (start 157.091967 45.63741) (end 156.811967 45.91741) (width 0.25) (layer "B.Cu") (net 2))
 (segment (start 160.056967 48.48441) (end 167.091967 48.48441) (width 0.4) (layer "B.Cu") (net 19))
 (segment (start 159.906967 48.33441) (end 160.056967 48.48441) (width 0.4) (layer "B.Cu") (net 19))
 (segment (start 167.091967 48.48441) (end 167.291967 48.28441) (width 0.4) (layer "B.Cu") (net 19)))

